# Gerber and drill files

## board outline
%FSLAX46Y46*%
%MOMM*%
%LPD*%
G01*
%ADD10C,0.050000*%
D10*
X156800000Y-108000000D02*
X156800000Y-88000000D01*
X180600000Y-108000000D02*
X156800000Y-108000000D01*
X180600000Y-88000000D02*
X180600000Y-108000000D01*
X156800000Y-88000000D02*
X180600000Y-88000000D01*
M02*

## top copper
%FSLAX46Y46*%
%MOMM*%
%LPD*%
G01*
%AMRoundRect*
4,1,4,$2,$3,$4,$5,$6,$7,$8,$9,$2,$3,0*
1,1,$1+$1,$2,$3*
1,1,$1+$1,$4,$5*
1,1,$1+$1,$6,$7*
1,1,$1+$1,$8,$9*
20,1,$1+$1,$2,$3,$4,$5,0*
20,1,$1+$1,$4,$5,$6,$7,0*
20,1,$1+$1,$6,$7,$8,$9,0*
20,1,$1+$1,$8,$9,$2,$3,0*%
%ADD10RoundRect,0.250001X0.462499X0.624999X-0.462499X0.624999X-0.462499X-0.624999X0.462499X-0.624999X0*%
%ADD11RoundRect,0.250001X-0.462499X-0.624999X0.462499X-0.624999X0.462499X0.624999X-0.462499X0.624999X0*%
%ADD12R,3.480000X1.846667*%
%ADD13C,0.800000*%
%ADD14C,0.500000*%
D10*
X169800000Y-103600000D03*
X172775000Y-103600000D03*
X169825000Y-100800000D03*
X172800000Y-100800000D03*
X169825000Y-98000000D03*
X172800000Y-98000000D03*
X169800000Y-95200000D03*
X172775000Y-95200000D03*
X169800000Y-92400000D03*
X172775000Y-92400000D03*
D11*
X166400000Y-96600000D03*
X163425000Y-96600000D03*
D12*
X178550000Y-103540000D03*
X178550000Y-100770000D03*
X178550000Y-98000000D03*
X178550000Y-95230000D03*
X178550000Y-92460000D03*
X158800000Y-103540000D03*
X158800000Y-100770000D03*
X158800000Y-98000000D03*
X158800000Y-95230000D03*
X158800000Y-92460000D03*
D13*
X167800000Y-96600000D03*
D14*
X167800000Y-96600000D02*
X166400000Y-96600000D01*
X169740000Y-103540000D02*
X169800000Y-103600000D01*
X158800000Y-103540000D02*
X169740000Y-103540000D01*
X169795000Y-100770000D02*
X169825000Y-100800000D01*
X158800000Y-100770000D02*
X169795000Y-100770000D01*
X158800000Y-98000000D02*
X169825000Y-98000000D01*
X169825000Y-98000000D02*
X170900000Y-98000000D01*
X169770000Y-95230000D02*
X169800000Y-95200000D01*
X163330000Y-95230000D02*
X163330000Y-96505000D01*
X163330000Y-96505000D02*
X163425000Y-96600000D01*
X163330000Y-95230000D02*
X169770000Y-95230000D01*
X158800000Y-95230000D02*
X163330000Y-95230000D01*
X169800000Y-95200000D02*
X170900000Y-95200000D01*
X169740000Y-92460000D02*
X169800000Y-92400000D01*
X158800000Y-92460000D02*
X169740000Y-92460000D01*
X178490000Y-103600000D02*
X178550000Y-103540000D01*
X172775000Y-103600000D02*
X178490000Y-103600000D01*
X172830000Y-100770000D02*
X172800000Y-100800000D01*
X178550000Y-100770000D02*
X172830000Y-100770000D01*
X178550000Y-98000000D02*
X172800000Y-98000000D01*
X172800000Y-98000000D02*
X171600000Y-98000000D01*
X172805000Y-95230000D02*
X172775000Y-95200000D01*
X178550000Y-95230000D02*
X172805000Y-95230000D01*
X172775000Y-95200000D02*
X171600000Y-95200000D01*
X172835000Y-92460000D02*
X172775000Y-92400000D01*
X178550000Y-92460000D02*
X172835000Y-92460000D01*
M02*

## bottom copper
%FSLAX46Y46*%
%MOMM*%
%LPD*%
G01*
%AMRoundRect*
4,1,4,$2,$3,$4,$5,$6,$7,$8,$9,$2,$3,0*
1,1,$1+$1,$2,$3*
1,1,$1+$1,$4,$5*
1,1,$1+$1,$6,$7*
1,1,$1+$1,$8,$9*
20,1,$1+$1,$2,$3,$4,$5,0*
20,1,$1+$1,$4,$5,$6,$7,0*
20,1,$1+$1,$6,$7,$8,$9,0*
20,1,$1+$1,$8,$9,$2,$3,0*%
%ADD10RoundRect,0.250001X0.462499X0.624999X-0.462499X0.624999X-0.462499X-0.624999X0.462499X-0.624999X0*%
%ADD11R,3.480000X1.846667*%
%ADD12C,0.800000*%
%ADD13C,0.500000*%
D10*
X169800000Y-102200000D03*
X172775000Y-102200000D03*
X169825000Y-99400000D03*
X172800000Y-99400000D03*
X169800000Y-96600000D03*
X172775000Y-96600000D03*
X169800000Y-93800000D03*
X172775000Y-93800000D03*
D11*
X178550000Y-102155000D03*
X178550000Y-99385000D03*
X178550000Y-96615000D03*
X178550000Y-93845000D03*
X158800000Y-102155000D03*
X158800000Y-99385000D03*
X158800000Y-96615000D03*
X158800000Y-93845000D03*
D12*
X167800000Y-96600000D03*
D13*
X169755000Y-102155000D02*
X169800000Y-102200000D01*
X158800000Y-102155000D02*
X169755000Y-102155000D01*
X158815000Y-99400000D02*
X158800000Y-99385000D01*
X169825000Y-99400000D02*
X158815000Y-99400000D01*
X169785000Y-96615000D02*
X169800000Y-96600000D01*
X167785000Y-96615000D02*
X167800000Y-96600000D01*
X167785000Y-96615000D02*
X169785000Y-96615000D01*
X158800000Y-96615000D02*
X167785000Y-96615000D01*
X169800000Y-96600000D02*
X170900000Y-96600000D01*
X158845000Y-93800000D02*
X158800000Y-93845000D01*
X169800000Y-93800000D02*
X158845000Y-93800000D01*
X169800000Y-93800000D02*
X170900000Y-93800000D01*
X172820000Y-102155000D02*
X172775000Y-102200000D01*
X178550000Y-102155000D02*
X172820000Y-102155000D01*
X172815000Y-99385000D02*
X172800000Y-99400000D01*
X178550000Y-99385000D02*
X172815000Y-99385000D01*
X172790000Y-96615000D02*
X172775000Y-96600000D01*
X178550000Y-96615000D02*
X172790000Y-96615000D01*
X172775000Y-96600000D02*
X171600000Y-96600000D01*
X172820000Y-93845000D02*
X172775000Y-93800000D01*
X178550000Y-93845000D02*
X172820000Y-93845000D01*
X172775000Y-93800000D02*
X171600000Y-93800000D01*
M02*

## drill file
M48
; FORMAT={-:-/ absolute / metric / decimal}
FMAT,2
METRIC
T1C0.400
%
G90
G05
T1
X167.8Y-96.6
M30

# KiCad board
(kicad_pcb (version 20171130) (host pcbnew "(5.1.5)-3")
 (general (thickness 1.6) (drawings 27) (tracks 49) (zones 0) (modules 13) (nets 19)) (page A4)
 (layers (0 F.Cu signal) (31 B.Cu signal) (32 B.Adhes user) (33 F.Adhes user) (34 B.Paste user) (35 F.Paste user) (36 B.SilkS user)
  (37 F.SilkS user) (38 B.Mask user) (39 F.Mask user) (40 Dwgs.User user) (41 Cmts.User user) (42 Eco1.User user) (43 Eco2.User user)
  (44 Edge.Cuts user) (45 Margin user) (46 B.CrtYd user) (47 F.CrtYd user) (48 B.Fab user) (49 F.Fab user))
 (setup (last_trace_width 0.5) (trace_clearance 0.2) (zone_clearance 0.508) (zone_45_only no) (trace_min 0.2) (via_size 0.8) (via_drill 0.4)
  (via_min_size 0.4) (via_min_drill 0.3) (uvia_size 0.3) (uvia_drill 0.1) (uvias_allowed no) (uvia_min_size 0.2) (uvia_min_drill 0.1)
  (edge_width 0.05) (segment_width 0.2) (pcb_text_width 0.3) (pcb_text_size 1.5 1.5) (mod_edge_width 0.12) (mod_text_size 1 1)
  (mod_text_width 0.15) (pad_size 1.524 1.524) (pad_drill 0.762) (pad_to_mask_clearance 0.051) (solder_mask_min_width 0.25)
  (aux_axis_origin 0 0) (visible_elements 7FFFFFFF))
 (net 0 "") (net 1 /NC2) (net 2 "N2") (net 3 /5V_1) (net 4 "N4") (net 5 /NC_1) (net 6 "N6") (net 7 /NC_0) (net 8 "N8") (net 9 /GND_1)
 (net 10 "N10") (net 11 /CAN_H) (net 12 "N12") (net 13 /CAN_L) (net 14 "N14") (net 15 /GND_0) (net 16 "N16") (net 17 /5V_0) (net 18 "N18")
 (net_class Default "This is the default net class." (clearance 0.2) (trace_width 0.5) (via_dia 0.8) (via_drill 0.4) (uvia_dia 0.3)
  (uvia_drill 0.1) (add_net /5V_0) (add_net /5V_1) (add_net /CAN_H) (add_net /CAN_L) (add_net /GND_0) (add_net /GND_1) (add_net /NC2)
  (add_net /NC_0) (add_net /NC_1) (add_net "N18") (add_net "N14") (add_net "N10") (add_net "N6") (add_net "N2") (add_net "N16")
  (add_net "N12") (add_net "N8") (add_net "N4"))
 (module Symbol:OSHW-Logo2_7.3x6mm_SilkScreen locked (layer F.Cu) (at 165.9 102.9)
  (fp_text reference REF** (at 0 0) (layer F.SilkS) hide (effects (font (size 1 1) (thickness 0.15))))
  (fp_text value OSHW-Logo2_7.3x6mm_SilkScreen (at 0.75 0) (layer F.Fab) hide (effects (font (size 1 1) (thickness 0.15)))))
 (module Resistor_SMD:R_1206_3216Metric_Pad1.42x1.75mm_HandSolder (layer F.Cu) (at 171.2875 103.6 180)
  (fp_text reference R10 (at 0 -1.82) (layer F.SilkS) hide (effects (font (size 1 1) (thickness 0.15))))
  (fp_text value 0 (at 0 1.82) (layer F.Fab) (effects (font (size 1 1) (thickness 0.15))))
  (pad 2 smd roundrect (at 1.4875 0 180) (size 1.425 1.75) (layers F.Cu F.Paste F.Mask) (roundrect_rratio 0.175439) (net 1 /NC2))
  (pad 1 smd roundrect (at -1.4875 0 180) (size 1.425 1.75) (layers F.Cu F.Paste F.Mask) (roundrect_rratio 0.175439) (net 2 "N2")))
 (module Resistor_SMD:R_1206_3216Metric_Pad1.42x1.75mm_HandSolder (layer B.Cu) (at 171.2875 102.2 180)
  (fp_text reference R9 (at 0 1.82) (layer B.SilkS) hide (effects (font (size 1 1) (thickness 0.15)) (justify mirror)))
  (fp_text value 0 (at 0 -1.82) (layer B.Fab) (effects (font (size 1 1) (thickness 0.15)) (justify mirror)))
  (pad 2 smd roundrect (at 1.4875 0 180) (size 1.425 1.75) (layers B.Cu B.Paste B.Mask) (roundrect_rratio 0.175439) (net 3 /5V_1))
  (pad 1 smd roundrect (at -1.4875 0 180) (size 1.425 1.75) (layers B.Cu B.Paste B.Mask) (roundrect_rratio 0.175439) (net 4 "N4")))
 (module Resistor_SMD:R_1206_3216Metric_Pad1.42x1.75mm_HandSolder (layer F.Cu) (at 171.3125 100.8 180)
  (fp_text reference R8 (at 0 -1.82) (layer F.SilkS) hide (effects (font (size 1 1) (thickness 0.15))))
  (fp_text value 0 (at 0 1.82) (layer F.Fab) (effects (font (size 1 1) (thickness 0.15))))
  (pad 2 smd roundrect (at 1.4875 0 180) (size 1.425 1.75) (layers F.Cu F.Paste F.Mask) (roundrect_rratio 0.175439) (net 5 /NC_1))
  (pad 1 smd roundrect (at -1.4875 0 180) (size 1.425 1.75) (layers F.Cu F.Paste F.Mask) (roundrect_rratio 0.175439) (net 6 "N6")))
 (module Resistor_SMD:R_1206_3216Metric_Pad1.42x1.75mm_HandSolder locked (layer B.Cu) (at 171.3125 99.4 180)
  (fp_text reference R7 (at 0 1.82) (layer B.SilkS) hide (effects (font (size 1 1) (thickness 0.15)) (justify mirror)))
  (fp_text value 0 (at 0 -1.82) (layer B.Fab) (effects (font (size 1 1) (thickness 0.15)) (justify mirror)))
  (pad 2 smd roundrect (at 1.4875 0 180) (size 1.425 1.75) (layers B.Cu B.Paste B.Mask) (roundrect_rratio 0.175439) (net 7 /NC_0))
  (pad 1 smd roundrect (at -1.4875 0 180) (size 1.425 1.75) (layers B.Cu B.Paste B.Mask) (roundrect_rratio 0.175439) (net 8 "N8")))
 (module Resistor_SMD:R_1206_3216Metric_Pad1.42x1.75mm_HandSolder (layer F.Cu) (at 171.3125 98 180)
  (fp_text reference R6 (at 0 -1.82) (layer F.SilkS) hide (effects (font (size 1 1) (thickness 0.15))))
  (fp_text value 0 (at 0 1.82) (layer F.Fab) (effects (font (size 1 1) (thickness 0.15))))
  (pad 2 smd roundrect (at 1.4875 0 180) (size 1.425 1.75) (layers F.Cu F.Paste F.Mask) (roundrect_rratio 0.175439) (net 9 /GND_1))
  (pad 1 smd roundrect (at -1.4875 0 180) (size 1.425 1.75) (layers F.Cu F.Paste F.Mask) (roundrect_rratio 0.175439) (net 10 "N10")))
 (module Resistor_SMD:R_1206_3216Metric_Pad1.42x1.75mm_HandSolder (layer B.Cu) (at 171.2875 96.6 180)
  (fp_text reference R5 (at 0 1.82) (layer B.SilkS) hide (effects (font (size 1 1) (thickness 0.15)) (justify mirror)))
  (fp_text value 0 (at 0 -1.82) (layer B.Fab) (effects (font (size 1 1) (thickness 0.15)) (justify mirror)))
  (pad 2 smd roundrect (at 1.4875 0 180) (size 1.425 1.75) (layers B.Cu B.Paste B.Mask) (roundrect_rratio 0.175439) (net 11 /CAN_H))
  (pad 1 smd roundrect (at -1.4875 0 180) (size 1.425 1.75) (layers B.Cu B.Paste B.Mask) (roundrect_rratio 0.175439) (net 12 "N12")))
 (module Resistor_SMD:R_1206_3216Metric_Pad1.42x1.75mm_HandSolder (layer F.Cu) (at 171.2875 95.2 180)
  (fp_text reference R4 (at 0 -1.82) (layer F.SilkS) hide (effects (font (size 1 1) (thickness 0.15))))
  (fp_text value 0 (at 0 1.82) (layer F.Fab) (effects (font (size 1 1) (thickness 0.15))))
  (pad 2 smd roundrect (at 1.4875 0 180) (size 1.425 1.75) (layers F.Cu F.Paste F.Mask) (roundrect_rratio 0.175439) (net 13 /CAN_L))
  (pad 1 smd roundrect (at -1.4875 0 180) (size 1.425 1.75) (layers F.Cu F.Paste F.Mask) (roundrect_rratio 0.175439) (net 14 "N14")))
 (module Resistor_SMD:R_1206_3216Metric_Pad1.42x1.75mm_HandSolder (layer B.Cu) (at 171.2875 93.8 180)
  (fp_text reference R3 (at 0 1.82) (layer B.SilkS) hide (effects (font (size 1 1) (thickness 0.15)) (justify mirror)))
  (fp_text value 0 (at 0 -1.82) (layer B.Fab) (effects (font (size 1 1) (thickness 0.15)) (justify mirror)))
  (pad 2 smd roundrect (at 1.4875 0 180) (size 1.425 1.75) (layers B.Cu B.Paste B.Mask) (roundrect_rratio 0.175439) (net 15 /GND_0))
  (pad 1 smd roundrect (at -1.4875 0 180) (size 1.425 1.75) (layers B.Cu B.Paste B.Mask) (roundrect_rratio 0.175439) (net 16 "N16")))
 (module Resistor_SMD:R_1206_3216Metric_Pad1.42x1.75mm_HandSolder (layer F.Cu) (at 171.2875 92.4 180)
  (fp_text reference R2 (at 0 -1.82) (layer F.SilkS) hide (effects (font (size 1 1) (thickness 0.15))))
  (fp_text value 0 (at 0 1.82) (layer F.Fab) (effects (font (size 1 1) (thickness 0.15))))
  (pad 2 smd roundrect (at 1.4875 0 180) (size 1.425 1.75) (layers F.Cu F.Paste F.Mask) (roundrect_rratio 0.175439) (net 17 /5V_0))
  (pad 1 smd roundrect (at -1.4875 0 180) (size 1.425 1.75) (layers F.Cu F.Paste F.Mask) (roundrect_rratio 0.175439) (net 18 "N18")))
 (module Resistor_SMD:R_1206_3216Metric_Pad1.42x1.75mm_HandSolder (layer F.Cu) (at 164.9125 96.6)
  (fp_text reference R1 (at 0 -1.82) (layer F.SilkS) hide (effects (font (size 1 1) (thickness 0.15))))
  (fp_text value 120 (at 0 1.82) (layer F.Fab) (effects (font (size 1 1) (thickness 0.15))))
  (pad 2 smd roundrect (at 1.4875 0) (size 1.425 1.75) (layers F.Cu F.Paste F.Mask) (roundrect_rratio 0.175439) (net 11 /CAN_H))
  (pad 1 smd roundrect (at -1.4875 0) (size 1.425 1.75) (layers F.Cu F.Paste F.Mask) (roundrect_rratio 0.175439) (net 13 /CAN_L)))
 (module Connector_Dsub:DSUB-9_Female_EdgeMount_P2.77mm (layer F.Cu) (at 178.55 98 90)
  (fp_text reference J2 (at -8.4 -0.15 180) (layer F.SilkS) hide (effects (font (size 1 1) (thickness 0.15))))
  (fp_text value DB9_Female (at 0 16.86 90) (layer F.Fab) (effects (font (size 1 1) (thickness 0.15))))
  (pad 9 smd rect (at -4.155 0 90) (size 1.846667 3.48) (layers B.Cu B.Paste B.Mask) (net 4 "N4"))
  (pad 8 smd rect (at -1.385 0 90) (size 1.846667 3.48) (layers B.Cu B.Paste B.Mask) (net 8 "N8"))
  (pad 7 smd rect (at 1.385 0 90) (size 1.846667 3.48) (layers B.Cu B.Paste B.Mask) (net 12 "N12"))
  (pad 6 smd rect (at 4.155 0 90) (size 1.846667 3.48) (layers B.Cu B.Paste B.Mask) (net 16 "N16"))
  (pad 5 smd rect (at -5.54 0 90) (size 1.846667 3.48) (layers F.Cu F.Paste F.Mask) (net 2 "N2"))
  (pad 4 smd rect (at -2.77 0 90) (size 1.846667 3.48) (layers F.Cu F.Paste F.Mask) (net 6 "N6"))
  (pad 3 smd rect (at 0 0 90) (size 1.846667 3.48) (layers F.Cu F.Paste F.Mask) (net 10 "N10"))
  (pad 2 smd rect (at 2.77 0 90) (size 1.846667 3.48) (layers F.Cu F.Paste F.Mask) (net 14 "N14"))
  (pad 1 smd rect (at 5.54 0 90) (size 1.846667 3.48) (layers F.Cu F.Paste F.Mask) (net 18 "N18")))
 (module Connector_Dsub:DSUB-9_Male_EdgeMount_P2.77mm (layer F.Cu) (at 158.8 98 270)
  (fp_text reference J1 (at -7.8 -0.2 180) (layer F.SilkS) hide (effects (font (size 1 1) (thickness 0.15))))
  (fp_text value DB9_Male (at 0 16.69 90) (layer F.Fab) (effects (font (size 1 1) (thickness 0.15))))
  (pad 9 smd rect (at 4.155 0 270) (size 1.846667 3.48) (layers B.Cu B.Paste B.Mask) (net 3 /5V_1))
  (pad 8 smd rect (at 1.385 0 270) (size 1.846667 3.48) (layers B.Cu B.Paste B.Mask) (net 7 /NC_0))
  (pad 7 smd rect (at -1.385 0 270) (size 1.846667 3.48) (layers B.Cu B.Paste B.Mask) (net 11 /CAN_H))
  (pad 6 smd rect (at -4.155 0 270) (size 1.846667 3.48) (layers B.Cu B.Paste B.Mask) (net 15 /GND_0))
  (pad 5 smd rect (at 5.54 0 270) (size 1.846667 3.48) (layers F.Cu F.Paste F.Mask) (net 1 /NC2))
  (pad 4 smd rect (at 2.77 0 270) (size 1.846667 3.48) (layers F.Cu F.Paste F.Mask) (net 5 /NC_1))
  (pad 3 smd rect (at 0 0 270) (size 1.846667 3.48) (layers F.Cu F.Paste F.Mask) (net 9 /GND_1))
  (pad 2 smd rect (at -2.77 0 270) (size 1.846667 3.48) (layers F.Cu F.Paste F.Mask) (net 13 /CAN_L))
  (pad 1 smd rect (at -5.54 0 270) (size 1.846667 3.48) (layers F.Cu F.Paste F.Mask) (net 17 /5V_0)))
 (gr_line (start 156.8 108) (end 156.8 88) (layer Edge.Cuts) (width 0.05))
 (gr_line (start 180.6 108) (end 156.8 108) (layer Edge.Cuts) (width 0.05))
 (gr_line (start 180.6 88) (end 180.6 108) (layer Edge.Cuts) (width 0.05))
 (gr_line (start 156.8 88) (end 180.6 88) (layer Edge.Cuts) (width 0.05))
 (segment (start 169.755 102.155) (end 169.8 102.2) (width 0.5) (layer B.Cu) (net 3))
 (segment (start 158.8 102.155) (end 169.755 102.155) (width 0.5) (layer B.Cu) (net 3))
 (segment (start 158.815 99.4) (end 158.8 99.385) (width 0.5) (layer B.Cu) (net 7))
 (segment (start 169.825 99.4) (end 158.815 99.4) (width 0.5) (layer B.Cu) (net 7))
 (segment (start 169.785 96.615) (end 169.8 96.6) (width 0.5) (layer B.Cu) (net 11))
 (segment (start 167.785 96.615) (end 167.8 96.6) (width 0.5) (layer B.Cu) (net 11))
 (segment (start 167.785 96.615) (end 169.785 96.615) (width 0.5) (layer B.Cu) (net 11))
 (via (at 167.8 96.6) (size 0.8) (drill 0.4) (layers F.Cu B.Cu) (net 11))
 (segment (start 158.8 96.615) (end 167.785 96.615) (width 0.5) (layer B.Cu) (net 11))
 (segment (start 167.8 96.6) (end 166.4 96.6) (width 0.5) (layer F.Cu) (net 11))
 (segment (start 169.8 96.6) (end 170.9 96.6) (width 0.5) (layer B.Cu) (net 11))
 (segment (start 158.845 93.8) (end 158.8 93.845) (width 0.5) (layer B.Cu) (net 15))
 (segment (start 169.8 93.8) (end 158.845 93.8) (width 0.5) (layer B.Cu) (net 15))
 (segment (start 169.8 93.8) (end 170.9 93.8) (width 0.5) (layer B.Cu) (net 15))
 (segment (start 169.74 103.54) (end 169.8 103.6) (width 0.5) (layer F.Cu) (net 1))
 (segment (start 158.8 103.54) (end 169.74 103.54) (width 0.5) (layer F.Cu) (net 1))
 (segment (start 169.795 100.77) (end 169.825 100.8) (width 0.5) (layer F.Cu) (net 5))
 (segment (start 158.8 100.77) (end 169.795 100.77) (width 0.5) (layer F.Cu) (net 5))
 (segment (start 158.8 98) (end 169.825 98) (width 0.5) (layer F.Cu) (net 9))
 (segment (start 169.825 98) (end 170.9 98) (width 0.5) (layer F.Cu) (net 9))
 (segment (start 169.77 95.23) (end 169.8 95.2) (width 0.5) (layer F.Cu) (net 13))
 (segment (start 163.33 95.23) (end 163.33 96.505) (width 0.5) (layer F.Cu) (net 13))
 (segment (start 163.33 96.505) (end 163.425 96.6) (width 0.5) (layer F.Cu) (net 13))
 (segment (start 163.33 95.23) (end 169.77 95.23) (width 0.5) (layer F.Cu) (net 13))
 (segment (start 158.8 95.23) (end 163.33 95.23) (width 0.5) (layer F.Cu) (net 13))
 (segment (start 169.8 95.2) (end 170.9 95.2) (width 0.5) (layer F.Cu) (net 13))
 (segment (start 169.74 92.46) (end 169.8 92.4) (width 0.5) (layer F.Cu) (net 17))
 (segment (start 158.8 92.46) (end 169.74 92.46) (width 0.5) (layer F.Cu) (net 17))
 (segment (start 172.82 102.155) (end 172.775 102.2) (width 0.5) (layer B.Cu) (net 4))
 (segment (start 178.55 102.155) (end 172.82 102.155) (width 0.5) (layer B.Cu) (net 4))
 (segment (start 172.815 99.385) (end 172.8 99.4) (width 0.5) (layer B.Cu) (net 8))
 (segment (start 178.55 99.385) (end 172.815 99.385) (width 0.5) (layer B.Cu) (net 8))
 (segment (start 172.79 96.615) (end 172.775 96.6) (width 0.5) (layer B.Cu) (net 12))
 (segment (start 178.55 96.615) (end 172.79 96.615) (width 0.5) (layer B.Cu) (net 12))
 (segment (start 172.775 96.6) (end 171.6 96.6) (width 0.5) (layer B.Cu) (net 12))
 (segment (start 172.82 93.845) (end 172.775 93.8) (width 0.5) (layer B.Cu) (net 16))
 (segment (start 178.55 93.845) (end 172.82 93.845) (width 0.5) (layer B.Cu) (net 16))
 (segment (start 172.775 93.8) (end 171.6 93.8) (width 0.5) (layer B.Cu) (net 16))
 (segment (start 178.49 103.6) (end 178.55 103.54) (width 0.5) (layer F.Cu) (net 2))
 (segment (start 172.775 103.6) (end 178.49 103.6) (width 0.5) (layer F.Cu) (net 2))
 (segment (start 172.83 100.77) (end 172.8 100.8) (width 0.5) (layer F.Cu) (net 6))
 (segment (start 178.55 100.77) (end 172.83 100.77) (width 0.5) (layer F.Cu) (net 6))
 (segment (start 178.55 98) (end 172.8 98) (width 0.5) (layer F.Cu) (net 10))
 (segment (start 172.8 98) (end 171.6 98) (width 0.5) (layer F.Cu) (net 10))
 (segment (start 172.805 95.23) (end 172.775 95.2) (width 0.5) (layer F.Cu) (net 14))
 (segment (start 178.55 95.23) (end 172.805 95.23) (width 0.5) (layer F.Cu) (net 14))
 (segment (start 172.775 95.2) (end 171.6 95.2) (width 0.5) (layer F.Cu) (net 14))
 (segment (start 172.835 92.46) (end 172.775 92.4) (width 0.5) (layer F.Cu) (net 18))
 (segment (start 178.55 92.46) (end 172.835 92.46) (width 0.5) (layer F.Cu) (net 18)))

